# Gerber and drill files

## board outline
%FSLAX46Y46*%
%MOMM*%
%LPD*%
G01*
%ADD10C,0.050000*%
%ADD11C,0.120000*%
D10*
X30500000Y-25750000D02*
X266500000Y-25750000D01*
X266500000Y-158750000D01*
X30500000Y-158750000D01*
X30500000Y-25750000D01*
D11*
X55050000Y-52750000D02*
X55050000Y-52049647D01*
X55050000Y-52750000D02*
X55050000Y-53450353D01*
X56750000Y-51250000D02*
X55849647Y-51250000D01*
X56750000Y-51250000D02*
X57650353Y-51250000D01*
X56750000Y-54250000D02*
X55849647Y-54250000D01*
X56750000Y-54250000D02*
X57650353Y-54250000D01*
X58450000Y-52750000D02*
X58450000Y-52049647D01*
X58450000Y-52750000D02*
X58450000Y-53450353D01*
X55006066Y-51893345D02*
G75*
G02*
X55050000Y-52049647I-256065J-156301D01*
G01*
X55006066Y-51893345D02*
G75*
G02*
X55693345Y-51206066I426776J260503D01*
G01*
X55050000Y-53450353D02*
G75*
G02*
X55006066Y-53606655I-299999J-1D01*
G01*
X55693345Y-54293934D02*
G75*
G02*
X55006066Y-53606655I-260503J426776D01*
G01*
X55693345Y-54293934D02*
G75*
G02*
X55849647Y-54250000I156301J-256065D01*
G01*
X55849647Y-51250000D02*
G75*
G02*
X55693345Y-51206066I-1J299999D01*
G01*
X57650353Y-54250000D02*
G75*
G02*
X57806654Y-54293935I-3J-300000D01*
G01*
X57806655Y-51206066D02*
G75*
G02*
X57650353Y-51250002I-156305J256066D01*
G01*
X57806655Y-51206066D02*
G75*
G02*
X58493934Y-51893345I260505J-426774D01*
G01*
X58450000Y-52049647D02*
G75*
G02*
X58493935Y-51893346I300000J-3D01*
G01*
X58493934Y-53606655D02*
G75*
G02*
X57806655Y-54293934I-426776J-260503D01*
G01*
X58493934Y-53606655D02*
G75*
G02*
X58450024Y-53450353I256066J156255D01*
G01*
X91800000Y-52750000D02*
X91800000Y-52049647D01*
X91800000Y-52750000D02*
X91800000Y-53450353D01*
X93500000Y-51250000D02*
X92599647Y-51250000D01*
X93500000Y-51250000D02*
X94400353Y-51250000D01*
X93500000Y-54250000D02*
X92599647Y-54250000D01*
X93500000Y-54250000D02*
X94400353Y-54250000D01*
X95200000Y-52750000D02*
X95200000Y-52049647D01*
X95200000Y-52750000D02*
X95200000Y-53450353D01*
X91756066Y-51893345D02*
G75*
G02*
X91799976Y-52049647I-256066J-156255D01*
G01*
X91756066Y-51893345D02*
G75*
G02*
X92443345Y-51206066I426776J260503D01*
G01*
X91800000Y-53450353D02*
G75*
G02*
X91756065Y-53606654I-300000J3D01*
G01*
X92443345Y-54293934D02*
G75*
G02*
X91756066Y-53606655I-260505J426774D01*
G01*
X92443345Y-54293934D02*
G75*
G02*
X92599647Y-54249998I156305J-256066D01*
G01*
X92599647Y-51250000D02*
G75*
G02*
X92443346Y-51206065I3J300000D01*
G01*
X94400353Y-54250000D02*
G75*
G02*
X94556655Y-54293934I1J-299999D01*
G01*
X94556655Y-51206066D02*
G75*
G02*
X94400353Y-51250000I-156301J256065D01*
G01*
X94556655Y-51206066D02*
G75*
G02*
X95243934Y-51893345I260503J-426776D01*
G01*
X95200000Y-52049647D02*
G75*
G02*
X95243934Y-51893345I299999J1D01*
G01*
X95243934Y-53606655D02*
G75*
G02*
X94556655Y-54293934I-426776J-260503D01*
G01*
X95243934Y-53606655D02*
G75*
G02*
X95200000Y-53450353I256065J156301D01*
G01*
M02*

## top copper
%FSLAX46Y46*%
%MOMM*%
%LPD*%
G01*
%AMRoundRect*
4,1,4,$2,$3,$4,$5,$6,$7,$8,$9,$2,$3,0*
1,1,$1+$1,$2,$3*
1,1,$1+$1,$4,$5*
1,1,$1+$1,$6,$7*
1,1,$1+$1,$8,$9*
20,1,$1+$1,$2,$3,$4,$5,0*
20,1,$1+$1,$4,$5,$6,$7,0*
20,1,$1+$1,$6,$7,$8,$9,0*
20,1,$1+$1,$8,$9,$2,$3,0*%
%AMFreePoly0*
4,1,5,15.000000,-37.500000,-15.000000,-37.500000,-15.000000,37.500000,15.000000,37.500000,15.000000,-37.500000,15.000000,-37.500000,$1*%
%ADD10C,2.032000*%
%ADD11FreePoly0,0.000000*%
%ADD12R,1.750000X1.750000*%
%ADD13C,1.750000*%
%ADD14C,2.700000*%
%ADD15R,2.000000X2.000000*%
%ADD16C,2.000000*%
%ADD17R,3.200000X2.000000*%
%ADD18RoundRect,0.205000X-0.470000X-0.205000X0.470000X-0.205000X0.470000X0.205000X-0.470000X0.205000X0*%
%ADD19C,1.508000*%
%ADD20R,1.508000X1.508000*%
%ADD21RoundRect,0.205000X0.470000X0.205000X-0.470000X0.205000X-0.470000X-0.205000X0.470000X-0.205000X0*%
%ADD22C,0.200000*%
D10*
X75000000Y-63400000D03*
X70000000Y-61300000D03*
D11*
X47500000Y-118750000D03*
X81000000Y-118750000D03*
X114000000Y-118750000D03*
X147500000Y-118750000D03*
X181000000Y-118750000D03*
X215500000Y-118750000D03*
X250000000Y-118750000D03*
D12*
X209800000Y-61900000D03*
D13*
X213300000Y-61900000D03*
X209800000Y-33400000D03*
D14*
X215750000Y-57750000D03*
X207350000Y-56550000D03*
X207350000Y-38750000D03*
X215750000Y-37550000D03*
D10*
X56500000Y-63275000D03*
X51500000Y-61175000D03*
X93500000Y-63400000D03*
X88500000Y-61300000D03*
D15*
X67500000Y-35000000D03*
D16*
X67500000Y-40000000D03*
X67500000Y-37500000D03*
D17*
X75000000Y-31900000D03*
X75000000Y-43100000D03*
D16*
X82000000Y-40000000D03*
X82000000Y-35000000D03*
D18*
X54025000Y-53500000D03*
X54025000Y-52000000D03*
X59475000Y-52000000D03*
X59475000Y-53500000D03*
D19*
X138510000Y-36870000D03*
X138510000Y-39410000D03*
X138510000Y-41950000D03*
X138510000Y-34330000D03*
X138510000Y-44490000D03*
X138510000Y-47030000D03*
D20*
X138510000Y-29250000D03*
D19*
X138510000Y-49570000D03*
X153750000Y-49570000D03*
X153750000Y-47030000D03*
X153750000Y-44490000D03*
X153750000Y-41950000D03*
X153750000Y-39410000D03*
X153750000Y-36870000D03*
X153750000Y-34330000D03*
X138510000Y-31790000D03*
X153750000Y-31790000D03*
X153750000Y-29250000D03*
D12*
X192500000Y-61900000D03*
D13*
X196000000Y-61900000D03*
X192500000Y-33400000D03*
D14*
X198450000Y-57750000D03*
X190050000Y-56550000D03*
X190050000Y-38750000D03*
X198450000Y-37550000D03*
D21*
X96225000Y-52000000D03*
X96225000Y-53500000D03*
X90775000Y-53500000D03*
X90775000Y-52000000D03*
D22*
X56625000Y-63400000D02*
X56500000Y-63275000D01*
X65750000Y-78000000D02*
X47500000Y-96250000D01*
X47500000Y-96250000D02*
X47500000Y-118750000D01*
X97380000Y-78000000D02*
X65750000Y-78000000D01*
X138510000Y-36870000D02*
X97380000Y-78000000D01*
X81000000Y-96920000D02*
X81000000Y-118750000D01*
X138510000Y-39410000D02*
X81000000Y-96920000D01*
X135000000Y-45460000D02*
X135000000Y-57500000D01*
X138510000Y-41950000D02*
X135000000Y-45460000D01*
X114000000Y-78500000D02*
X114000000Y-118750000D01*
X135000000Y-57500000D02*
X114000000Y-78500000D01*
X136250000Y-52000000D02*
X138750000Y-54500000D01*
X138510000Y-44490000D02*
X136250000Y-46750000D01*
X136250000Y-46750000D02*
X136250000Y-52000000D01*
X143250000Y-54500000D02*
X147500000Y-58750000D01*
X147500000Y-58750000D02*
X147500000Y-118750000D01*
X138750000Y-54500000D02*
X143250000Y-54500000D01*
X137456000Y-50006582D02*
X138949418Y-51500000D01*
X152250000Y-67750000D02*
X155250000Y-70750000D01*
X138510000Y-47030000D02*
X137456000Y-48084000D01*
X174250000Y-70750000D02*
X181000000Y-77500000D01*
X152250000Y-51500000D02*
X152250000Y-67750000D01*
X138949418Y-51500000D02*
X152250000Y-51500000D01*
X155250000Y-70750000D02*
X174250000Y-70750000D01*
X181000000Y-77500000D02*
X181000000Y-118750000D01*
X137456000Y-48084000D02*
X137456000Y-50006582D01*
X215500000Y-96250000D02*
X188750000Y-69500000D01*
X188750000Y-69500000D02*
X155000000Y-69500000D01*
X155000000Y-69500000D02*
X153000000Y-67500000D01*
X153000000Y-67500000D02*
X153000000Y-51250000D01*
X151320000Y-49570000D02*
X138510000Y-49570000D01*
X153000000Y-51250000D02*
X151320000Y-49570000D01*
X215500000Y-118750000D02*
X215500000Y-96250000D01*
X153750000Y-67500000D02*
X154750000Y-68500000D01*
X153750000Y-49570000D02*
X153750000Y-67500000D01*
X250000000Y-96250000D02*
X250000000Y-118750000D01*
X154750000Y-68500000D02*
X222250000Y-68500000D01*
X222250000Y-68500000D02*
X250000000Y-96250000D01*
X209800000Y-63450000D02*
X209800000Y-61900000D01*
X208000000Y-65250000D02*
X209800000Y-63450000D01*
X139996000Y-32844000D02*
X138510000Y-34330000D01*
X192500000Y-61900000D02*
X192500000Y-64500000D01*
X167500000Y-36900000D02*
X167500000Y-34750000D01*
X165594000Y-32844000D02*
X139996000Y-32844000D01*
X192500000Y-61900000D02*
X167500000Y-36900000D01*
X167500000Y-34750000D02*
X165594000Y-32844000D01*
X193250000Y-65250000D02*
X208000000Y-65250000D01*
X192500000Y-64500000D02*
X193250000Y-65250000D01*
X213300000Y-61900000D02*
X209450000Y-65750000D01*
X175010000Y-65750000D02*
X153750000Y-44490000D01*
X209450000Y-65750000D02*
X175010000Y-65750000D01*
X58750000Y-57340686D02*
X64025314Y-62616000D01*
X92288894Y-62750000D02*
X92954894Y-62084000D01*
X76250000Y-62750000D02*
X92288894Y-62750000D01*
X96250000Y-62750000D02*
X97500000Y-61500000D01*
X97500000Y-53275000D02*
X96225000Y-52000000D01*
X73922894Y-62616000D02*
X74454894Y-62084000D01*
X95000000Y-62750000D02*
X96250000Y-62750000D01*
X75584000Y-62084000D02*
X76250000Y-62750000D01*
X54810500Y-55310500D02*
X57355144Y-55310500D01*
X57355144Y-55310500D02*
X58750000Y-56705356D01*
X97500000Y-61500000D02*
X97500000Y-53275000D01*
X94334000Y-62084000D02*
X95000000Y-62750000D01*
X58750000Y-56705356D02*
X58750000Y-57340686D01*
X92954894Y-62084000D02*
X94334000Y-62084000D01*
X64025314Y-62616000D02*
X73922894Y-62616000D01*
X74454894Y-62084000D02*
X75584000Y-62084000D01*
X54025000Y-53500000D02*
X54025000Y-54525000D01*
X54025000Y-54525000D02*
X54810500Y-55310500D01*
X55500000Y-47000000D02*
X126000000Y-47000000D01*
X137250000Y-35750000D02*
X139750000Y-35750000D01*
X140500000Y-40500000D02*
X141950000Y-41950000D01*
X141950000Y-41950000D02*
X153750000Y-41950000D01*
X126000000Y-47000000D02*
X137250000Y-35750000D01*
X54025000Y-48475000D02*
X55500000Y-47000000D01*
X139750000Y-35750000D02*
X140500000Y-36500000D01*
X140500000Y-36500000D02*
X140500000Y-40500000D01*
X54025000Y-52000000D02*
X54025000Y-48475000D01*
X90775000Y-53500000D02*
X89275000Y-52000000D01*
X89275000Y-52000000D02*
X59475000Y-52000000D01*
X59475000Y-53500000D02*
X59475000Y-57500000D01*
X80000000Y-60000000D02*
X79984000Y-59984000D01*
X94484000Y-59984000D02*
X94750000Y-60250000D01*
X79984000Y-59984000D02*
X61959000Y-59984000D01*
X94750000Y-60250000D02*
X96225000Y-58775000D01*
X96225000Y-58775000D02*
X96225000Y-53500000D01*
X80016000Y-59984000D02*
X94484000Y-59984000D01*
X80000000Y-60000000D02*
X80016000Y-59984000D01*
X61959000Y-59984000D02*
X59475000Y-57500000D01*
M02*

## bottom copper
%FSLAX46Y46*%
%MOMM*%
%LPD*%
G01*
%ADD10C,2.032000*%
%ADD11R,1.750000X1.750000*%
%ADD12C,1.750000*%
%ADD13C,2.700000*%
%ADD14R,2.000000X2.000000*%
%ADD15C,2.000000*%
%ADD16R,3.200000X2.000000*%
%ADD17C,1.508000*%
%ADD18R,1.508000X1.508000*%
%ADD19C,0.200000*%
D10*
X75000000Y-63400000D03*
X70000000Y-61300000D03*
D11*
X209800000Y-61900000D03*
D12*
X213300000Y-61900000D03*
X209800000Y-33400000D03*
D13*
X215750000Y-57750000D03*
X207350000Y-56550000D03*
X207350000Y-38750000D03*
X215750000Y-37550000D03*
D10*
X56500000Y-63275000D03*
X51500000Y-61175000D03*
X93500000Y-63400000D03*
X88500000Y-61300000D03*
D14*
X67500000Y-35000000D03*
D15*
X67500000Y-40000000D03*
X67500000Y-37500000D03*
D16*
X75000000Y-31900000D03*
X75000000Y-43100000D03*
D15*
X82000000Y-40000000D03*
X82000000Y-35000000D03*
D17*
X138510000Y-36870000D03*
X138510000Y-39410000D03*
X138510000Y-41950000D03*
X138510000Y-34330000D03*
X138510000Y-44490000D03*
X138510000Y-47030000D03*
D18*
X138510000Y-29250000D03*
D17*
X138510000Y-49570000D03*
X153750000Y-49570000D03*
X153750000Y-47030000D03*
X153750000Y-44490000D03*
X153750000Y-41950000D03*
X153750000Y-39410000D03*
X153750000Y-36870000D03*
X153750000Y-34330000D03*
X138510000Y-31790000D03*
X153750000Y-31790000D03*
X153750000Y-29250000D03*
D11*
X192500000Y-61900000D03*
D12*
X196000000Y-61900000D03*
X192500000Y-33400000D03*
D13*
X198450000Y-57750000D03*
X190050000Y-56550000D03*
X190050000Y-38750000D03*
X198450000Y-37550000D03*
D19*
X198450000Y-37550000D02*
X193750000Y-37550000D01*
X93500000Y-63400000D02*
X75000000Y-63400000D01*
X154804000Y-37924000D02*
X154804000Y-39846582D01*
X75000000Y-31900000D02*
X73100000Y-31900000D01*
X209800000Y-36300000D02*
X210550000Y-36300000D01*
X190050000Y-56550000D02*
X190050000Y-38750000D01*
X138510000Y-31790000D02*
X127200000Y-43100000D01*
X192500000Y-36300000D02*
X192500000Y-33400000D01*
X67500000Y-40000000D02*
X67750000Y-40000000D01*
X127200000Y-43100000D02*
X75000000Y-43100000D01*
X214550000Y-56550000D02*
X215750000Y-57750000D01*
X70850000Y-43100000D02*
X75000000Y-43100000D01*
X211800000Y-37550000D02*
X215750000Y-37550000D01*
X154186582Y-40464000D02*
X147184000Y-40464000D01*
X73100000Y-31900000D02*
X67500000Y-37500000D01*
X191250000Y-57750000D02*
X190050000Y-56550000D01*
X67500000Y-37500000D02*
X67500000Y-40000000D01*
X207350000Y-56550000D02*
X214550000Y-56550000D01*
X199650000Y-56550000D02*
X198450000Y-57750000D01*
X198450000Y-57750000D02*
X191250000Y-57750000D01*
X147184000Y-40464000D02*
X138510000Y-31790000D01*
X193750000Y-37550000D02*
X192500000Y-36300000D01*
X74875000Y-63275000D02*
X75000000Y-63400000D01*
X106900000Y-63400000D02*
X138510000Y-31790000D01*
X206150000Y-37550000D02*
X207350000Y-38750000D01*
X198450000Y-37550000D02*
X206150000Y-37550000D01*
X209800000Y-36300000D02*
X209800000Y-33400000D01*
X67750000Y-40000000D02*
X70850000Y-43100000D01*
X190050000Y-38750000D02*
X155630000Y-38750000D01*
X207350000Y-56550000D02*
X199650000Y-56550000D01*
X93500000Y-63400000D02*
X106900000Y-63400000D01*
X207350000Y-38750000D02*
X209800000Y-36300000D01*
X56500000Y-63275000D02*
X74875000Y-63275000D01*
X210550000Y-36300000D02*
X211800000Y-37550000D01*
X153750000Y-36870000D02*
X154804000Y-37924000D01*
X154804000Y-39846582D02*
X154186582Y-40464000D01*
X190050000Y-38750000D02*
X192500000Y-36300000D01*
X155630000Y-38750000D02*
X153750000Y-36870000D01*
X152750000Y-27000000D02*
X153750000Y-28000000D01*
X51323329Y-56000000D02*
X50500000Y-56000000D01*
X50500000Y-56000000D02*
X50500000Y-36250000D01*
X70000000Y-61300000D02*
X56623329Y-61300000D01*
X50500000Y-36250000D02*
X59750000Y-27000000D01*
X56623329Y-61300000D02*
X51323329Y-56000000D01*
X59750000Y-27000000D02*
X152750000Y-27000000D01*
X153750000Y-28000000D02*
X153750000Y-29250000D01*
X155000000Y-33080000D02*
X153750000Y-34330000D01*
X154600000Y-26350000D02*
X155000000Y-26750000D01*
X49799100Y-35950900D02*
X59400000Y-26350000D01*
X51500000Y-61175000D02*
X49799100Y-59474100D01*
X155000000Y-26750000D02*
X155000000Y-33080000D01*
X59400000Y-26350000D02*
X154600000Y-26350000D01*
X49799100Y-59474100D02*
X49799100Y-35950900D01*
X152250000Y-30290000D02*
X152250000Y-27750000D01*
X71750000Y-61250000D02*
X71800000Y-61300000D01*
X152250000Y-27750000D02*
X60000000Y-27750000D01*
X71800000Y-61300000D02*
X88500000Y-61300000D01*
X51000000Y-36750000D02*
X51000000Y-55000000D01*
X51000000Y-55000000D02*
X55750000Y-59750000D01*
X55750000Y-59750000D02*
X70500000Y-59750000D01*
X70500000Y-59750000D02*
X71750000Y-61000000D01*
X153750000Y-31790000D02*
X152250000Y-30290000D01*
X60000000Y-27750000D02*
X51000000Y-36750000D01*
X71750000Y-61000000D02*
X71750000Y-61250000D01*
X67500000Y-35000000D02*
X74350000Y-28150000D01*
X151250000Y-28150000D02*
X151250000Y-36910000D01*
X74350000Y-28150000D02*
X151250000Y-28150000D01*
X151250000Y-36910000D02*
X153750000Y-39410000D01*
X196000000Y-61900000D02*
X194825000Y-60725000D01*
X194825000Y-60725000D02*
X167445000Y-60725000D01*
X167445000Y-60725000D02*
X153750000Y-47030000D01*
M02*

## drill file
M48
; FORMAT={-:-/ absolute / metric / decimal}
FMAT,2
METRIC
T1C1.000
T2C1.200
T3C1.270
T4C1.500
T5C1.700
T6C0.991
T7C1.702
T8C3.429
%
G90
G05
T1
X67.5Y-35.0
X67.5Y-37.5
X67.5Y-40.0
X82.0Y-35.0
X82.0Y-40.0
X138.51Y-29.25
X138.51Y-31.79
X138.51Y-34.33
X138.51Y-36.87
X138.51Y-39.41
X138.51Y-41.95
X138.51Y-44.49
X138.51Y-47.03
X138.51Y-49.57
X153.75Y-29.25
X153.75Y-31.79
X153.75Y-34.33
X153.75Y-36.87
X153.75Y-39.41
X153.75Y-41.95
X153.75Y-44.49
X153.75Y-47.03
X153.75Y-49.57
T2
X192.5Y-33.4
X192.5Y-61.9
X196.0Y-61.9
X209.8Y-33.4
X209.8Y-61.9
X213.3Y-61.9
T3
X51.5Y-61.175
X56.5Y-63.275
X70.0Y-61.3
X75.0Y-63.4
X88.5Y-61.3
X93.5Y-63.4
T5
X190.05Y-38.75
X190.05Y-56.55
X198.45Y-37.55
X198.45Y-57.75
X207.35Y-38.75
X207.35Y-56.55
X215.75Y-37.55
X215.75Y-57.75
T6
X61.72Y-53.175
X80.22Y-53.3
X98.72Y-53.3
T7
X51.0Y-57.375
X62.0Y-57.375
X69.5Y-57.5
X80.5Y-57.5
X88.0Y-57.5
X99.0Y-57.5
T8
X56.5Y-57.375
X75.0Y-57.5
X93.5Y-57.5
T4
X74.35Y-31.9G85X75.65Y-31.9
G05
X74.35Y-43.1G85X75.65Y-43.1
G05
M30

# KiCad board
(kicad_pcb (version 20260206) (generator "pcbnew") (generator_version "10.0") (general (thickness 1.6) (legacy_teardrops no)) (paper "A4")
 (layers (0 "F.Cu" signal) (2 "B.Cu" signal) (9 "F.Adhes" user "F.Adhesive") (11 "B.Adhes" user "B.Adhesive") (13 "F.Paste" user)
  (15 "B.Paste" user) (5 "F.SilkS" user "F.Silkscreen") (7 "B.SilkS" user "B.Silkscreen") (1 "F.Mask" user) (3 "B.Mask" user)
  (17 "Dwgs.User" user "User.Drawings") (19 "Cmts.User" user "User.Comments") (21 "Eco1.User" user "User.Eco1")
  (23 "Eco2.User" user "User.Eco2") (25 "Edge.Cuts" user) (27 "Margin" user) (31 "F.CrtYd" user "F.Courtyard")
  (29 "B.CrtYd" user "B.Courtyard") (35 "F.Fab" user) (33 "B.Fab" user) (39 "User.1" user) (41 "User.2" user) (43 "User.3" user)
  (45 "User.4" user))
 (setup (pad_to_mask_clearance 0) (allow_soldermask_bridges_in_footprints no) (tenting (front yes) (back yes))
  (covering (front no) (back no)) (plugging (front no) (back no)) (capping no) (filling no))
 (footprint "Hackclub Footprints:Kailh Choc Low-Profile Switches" (layer "F.Cu") (at 75 57.5)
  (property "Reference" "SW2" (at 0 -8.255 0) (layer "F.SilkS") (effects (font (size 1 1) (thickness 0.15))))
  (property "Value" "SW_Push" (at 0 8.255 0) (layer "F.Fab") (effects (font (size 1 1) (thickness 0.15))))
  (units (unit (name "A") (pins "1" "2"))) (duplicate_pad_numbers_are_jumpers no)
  (pad "" np_thru_hole circle (at -5.5 0) (size 1.7018 1.7018) (drill 1.7018) (layers "*.Cu" "*.Mask"))
  (pad "" np_thru_hole circle (at 0 0) (size 3.429 3.429) (drill 3.429) (layers "*.Cu" "*.Mask"))
  (pad "" np_thru_hole circle (at 5.22 -4.2) (size 0.9906 0.9906) (drill 0.9906) (layers "*.Cu" "*.Mask"))
  (pad "" np_thru_hole circle (at 5.5 0) (size 1.7018 1.7018) (drill 1.7018) (layers "*.Cu" "*.Mask"))
  (pad "1" thru_hole circle (at 0 5.9) (size 2.032 2.032) (drill 1.27) (layers "*.Cu" "*.Mask") (remove_unused_layers no) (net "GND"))
  (pad "2" thru_hole circle (at -5 3.8) (size 2.032 2.032) (drill 1.27) (layers "*.Cu" "*.Mask") (remove_unused_layers no) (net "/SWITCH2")))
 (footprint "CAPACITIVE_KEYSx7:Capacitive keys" (layer "F.Cu") (at 147.5 81.25)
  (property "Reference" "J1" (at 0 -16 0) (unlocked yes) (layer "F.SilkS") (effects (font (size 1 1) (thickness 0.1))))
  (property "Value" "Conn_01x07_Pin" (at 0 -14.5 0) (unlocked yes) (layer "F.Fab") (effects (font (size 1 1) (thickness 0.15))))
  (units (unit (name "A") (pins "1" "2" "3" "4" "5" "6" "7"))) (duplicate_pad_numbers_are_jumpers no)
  (pad "1" smd custom (at -100 37.5) (size 30 75) (layers "F.Cu" "F.Mask" "F.Paste") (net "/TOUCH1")
   (options (clearance outline) (anchor rect)) (primitives))
  (pad "2" smd custom (at -66.5 37.5) (size 30 75) (layers "F.Cu" "F.Mask" "F.Paste") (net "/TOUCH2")
   (options (clearance outline) (anchor rect)) (primitives))
  (pad "3" smd custom (at -33.5 37.5) (size 30 75) (layers "F.Cu" "F.Mask" "F.Paste") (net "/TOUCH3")
   (options (clearance outline) (anchor rect)) (primitives))
  (pad "4" smd custom (at 0 37.5) (size 30 75) (layers "F.Cu" "F.Mask" "F.Paste") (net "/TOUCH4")
   (options (clearance outline) (anchor rect)) (primitives))
  (pad "5" smd custom (at 33.5 37.5) (size 30 75) (layers "F.Cu" "F.Mask" "F.Paste") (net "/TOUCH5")
   (options (clearance outline) (anchor rect)) (primitives))
  (pad "6" smd custom (at 68 37.5) (size 30 75) (layers "F.Cu" "F.Mask" "F.Paste") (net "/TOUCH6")
   (options (clearance outline) (anchor rect)) (primitives))
  (pad "7" smd custom (at 102.5 37.5) (size 30 75) (layers "F.Cu" "F.Mask" "F.Paste") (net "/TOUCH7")
   (options (clearance outline) (anchor rect)) (primitives)))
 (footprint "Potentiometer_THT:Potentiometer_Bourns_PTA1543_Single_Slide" (layer "F.Cu") (at 209.8 61.9 90)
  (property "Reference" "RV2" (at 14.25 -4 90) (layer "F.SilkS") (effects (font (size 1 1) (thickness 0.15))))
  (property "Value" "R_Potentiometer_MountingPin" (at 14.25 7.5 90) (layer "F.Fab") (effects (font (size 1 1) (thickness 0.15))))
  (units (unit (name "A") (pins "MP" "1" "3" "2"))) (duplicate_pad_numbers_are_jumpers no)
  (pad "1" thru_hole rect (at 0 0 90) (size 1.75 1.75) (drill 1.2) (layers "*.Cu" "*.Mask") (remove_unused_layers no) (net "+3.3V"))
  (pad "2" thru_hole circle (at 0 3.5 90) (size 1.75 1.75) (drill 1.2) (layers "*.Cu" "*.Mask") (remove_unused_layers no) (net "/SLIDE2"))
  (pad "3" thru_hole circle (at 28.5 0 90) (size 1.75 1.75) (drill 1.2) (layers "*.Cu" "*.Mask") (remove_unused_layers no) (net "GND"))
  (pad "MP" thru_hole circle (at 4.15 5.95 90) (size 2.7 2.7) (drill 1.7) (layers "*.Cu" "*.Mask") (remove_unused_layers no) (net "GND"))
  (pad "MP" thru_hole circle (at 5.35 -2.45 90) (size 2.7 2.7) (drill 1.7) (layers "*.Cu" "*.Mask") (remove_unused_layers no) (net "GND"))
  (pad "MP" thru_hole circle (at 23.15 -2.45 90) (size 2.7 2.7) (drill 1.7) (layers "*.Cu" "*.Mask") (remove_unused_layers no) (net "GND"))
  (pad "MP" thru_hole circle (at 24.35 5.95 90) (size 2.7 2.7) (drill 1.7) (layers "*.Cu" "*.Mask") (remove_unused_layers no) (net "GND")))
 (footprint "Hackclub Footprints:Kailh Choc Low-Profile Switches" (layer "F.Cu") (at 56.5 57.375)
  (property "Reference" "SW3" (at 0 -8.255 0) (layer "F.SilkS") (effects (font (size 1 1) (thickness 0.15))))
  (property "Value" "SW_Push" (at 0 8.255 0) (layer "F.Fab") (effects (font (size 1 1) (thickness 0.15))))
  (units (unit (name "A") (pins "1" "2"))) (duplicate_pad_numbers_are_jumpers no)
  (pad "" np_thru_hole circle (at -5.5 0) (size 1.7018 1.7018) (drill 1.7018) (layers "*.Cu" "*.Mask"))
  (pad "" np_thru_hole circle (at 0 0) (size 3.429 3.429) (drill 3.429) (layers "*.Cu" "*.Mask"))
  (pad "" np_thru_hole circle (at 5.22 -4.2) (size 0.9906 0.9906) (drill 0.9906) (layers "*.Cu" "*.Mask"))
  (pad "" np_thru_hole circle (at 5.5 0) (size 1.7018 1.7018) (drill 1.7018) (layers "*.Cu" "*.Mask"))
  (pad "1" thru_hole circle (at 0 5.9) (size 2.032 2.032) (drill 1.27) (layers "*.Cu" "*.Mask") (remove_unused_layers no) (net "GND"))
  (pad "2" thru_hole circle (at -5 3.8) (size 2.032 2.032) (drill 1.27) (layers "*.Cu" "*.Mask") (remove_unused_layers no) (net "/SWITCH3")))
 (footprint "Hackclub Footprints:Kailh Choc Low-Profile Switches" (layer "F.Cu") (at 93.5 57.5)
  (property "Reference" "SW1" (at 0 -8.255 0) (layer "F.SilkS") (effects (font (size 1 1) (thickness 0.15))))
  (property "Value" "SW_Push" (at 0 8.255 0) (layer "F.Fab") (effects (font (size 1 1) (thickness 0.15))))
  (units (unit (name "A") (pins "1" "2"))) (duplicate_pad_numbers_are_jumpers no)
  (pad "" np_thru_hole circle (at -5.5 0) (size 1.7018 1.7018) (drill 1.7018) (layers "*.Cu" "*.Mask"))
  (pad "" np_thru_hole circle (at 0 0) (size 3.429 3.429) (drill 3.429) (layers "*.Cu" "*.Mask"))
  (pad "" np_thru_hole circle (at 5.22 -4.2) (size 0.9906 0.9906) (drill 0.9906) (layers "*.Cu" "*.Mask"))
  (pad "" np_thru_hole circle (at 5.5 0) (size 1.7018 1.7018) (drill 1.7018) (layers "*.Cu" "*.Mask"))
  (pad "1" thru_hole circle (at 0 5.9) (size 2.032 2.032) (drill 1.27) (layers "*.Cu" "*.Mask") (remove_unused_layers no) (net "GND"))
  (pad "2" thru_hole circle (at -5 3.8) (size 2.032 2.032) (drill 1.27) (layers "*.Cu" "*.Mask") (remove_unused_layers no) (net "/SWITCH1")))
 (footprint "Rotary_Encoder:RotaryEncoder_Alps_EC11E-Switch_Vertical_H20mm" (layer "F.Cu") (at 67.5 35)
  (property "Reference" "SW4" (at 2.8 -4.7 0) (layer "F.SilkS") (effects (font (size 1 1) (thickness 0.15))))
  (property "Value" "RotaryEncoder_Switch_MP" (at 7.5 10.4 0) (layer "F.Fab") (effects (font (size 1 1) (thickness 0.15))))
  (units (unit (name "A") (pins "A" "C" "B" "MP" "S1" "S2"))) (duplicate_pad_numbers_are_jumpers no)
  (pad "A" thru_hole rect (at 0 0) (size 2 2) (drill 1) (layers "*.Cu" "*.Mask") (remove_unused_layers no) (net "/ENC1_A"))
  (pad "B" thru_hole circle (at 0 5) (size 2 2) (drill 1) (layers "*.Cu" "*.Mask") (remove_unused_layers no) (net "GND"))
  (pad "C" thru_hole circle (at 0 2.5) (size 2 2) (drill 1) (layers "*.Cu" "*.Mask") (remove_unused_layers no) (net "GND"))
  (pad "MP" thru_hole rect (at 7.5 -3.1) (size 3.2 2) (drill oval 2.8 1.5) (layers "*.Cu" "*.Mask") (remove_unused_layers no) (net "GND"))
  (pad "MP" thru_hole rect (at 7.5 8.1) (size 3.2 2) (drill oval 2.8 1.5) (layers "*.Cu" "*.Mask") (remove_unused_layers no) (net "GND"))
  (pad "S1" thru_hole circle (at 14.5 5) (size 2 2) (drill 1) (layers "*.Cu" "*.Mask") (remove_unused_layers no)
   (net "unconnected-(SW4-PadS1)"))
  (pad "S2" thru_hole circle (at 14.5 0) (size 2 2) (drill 1) (layers "*.Cu" "*.Mask") (remove_unused_layers no)
   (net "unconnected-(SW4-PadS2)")))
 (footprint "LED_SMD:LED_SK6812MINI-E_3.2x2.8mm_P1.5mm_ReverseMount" (layer "F.Cu") (at 56.75 52.75)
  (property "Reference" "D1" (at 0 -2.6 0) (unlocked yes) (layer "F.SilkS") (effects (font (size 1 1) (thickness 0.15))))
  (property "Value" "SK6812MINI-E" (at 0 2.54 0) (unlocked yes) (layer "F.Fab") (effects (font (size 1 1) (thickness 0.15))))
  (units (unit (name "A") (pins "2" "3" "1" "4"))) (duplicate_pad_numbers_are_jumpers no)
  (fp_line (start -1.7 0) (end -1.7 -0.700353) (stroke (width 0.12) (type solid)) (layer "Edge.Cuts"))
  (fp_line (start -1.7 0) (end -1.7 0.700353) (stroke (width 0.12) (type solid)) (layer "Edge.Cuts"))
  (fp_line (start 0 -1.5) (end -0.900353 -1.5) (stroke (width 0.12) (type solid)) (layer "Edge.Cuts"))
  (fp_line (start 0 -1.5) (end 0.900353 -1.5) (stroke (width 0.12) (type solid)) (layer "Edge.Cuts"))
  (fp_line (start 0 1.5) (end -0.900353 1.5) (stroke (width 0.12) (type solid)) (layer "Edge.Cuts"))
  (fp_line (start 0 1.5) (end 0.900353 1.5) (stroke (width 0.12) (type solid)) (layer "Edge.Cuts"))
  (fp_line (start 1.7 0) (end 1.7 -0.700353) (stroke (width 0.12) (type solid)) (layer "Edge.Cuts"))
  (fp_line (start 1.7 0) (end 1.7 0.700353) (stroke (width 0.12) (type solid)) (layer "Edge.Cuts"))
  (fp_arc (start -1.743934 -0.856655) (mid -1.711192 -0.781532) (end -1.7 -0.700353) (stroke (width 0.12) (type solid)) (layer "Edge.Cuts"))
  (fp_arc (start -1.743934 -0.856655) (mid -1.670711 -1.470711) (end -1.056655 -1.543934) (stroke (width 0.12) (type solid))
   (layer "Edge.Cuts"))
  (fp_arc (start -1.7 0.700353) (mid -1.711192 0.781532) (end -1.743934 0.856655) (stroke (width 0.12) (type solid)) (layer "Edge.Cuts"))
  (fp_arc (start -1.056655 1.543934) (mid -1.670711 1.470711) (end -1.743934 0.856655) (stroke (width 0.12) (type solid))
   (layer "Edge.Cuts"))
  (fp_arc (start -1.056655 1.543934) (mid -0.981532 1.511192) (end -0.900353 1.5) (stroke (width 0.12) (type solid)) (layer "Edge.Cuts"))
  (fp_arc (start -0.900353 -1.5) (mid -0.981532 -1.511192) (end -1.056655 -1.543934) (stroke (width 0.12) (type solid)) (layer "Edge.Cuts"))
  (fp_arc (start 0.900353 1.5) (mid 0.981532 1.511192) (end 1.056655 1.543934) (stroke (width 0.12) (type solid)) (layer "Edge.Cuts"))
  (fp_arc (start 1.056655 -1.543934) (mid 0.981532 -1.511192) (end 0.900353 -1.5) (stroke (width 0.12) (type solid)) (layer "Edge.Cuts"))
  (fp_arc (start 1.056655 -1.543934) (mid 1.670711 -1.470711) (end 1.743934 -0.856655) (stroke (width 0.12) (type solid))
   (layer "Edge.Cuts"))
  (fp_arc (start 1.7 -0.700353) (mid 1.711192 -0.781532) (end 1.743934 -0.856655) (stroke (width 0.12) (type solid)) (layer "Edge.Cuts"))
  (fp_arc (start 1.743934 0.856655) (mid 1.670711 1.470711) (end 1.056655 1.543934) (stroke (width 0.12) (type solid)) (layer "Edge.Cuts"))
  (fp_arc (start 1.743934 0.856655) (mid 1.711192 0.781532) (end 1.7 0.700353) (stroke (width 0.12) (type solid)) (layer "Edge.Cuts"))
  (pad "1" smd roundrect (at -2.725 0.75) (size 1.35 0.82) (layers "F.Cu" "F.Mask" "F.Paste") (roundrect_rratio 0.25) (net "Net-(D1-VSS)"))
  (pad "2" smd roundrect (at -2.725 -0.75) (size 1.35 0.82) (layers "F.Cu" "F.Mask" "F.Paste") (roundrect_rratio 0.25) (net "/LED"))
  (pad "3" smd roundrect (at 2.725 -0.75) (size 1.35 0.82) (layers "F.Cu" "F.Mask" "F.Paste") (roundrect_rratio 0.25) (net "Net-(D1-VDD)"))
  (pad "4" smd roundrect (at 2.725 0.75) (size 1.35 0.82) (layers "F.Cu" "F.Mask" "F.Paste") (roundrect_rratio 0.25) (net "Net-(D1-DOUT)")))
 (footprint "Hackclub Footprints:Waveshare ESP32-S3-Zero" (layer "F.Cu") (at 146.13 39.41)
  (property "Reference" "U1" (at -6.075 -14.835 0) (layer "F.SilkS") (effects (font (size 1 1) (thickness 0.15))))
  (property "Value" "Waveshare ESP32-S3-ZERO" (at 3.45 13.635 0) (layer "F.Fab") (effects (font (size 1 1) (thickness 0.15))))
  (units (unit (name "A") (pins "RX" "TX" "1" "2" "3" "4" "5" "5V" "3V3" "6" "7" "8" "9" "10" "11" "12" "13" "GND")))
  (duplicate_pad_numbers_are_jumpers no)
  (pad "1" thru_hole circle (at -7.62 -2.54) (size 1.508 1.508) (drill 1) (layers "*.Cu" "*.Mask") (remove_unused_layers no) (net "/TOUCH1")
   (solder_mask_margin 0.102))
  (pad "2" thru_hole circle (at -7.62 0) (size 1.508 1.508) (drill 1) (layers "*.Cu" "*.Mask") (remove_unused_layers no) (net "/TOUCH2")
   (solder_mask_margin 0.102))
  (pad "3" thru_hole circle (at -7.62 2.54) (size 1.508 1.508) (drill 1) (layers "*.Cu" "*.Mask") (remove_unused_layers no) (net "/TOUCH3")
   (solder_mask_margin 0.102))
  (pad "3V3" thru_hole circle (at -7.62 -5.08) (size 1.508 1.508) (drill 1) (layers "*.Cu" "*.Mask") (remove_unused_layers no) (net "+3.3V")
   (solder_mask_margin 0.102))
  (pad "4" thru_hole circle (at -7.62 5.08) (size 1.508 1.508) (drill 1) (layers "*.Cu" "*.Mask") (remove_unused_layers no) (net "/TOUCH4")
   (solder_mask_margin 0.102))
  (pad "5" thru_hole circle (at -7.62 7.62) (size 1.508 1.508) (drill 1) (layers "*.Cu" "*.Mask") (remove_unused_layers no) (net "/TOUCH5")
   (solder_mask_margin 0.102))
  (pad "5V" thru_hole rect (at -7.62 -10.16) (size 1.508 1.508) (drill 1) (layers "*.Cu" "*.Mask") (remove_unused_layers no) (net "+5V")
   (solder_mask_margin 0.102))
  (pad "6" thru_hole circle (at -7.62 10.16) (size 1.508 1.508) (drill 1) (layers "*.Cu" "*.Mask") (remove_unused_layers no) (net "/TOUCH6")
   (solder_mask_margin 0.102))
  (pad "7" thru_hole circle (at 7.62 10.16) (size 1.508 1.508) (drill 1) (layers "*.Cu" "*.Mask") (remove_unused_layers no) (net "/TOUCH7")
   (solder_mask_margin 0.102))
  (pad "8" thru_hole circle (at 7.62 7.62) (size 1.508 1.508) (drill 1) (layers "*.Cu" "*.Mask") (remove_unused_layers no) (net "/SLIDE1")
   (solder_mask_margin 0.102))
  (pad "9" thru_hole circle (at 7.62 5.08) (size 1.508 1.508) (drill 1) (layers "*.Cu" "*.Mask") (remove_unused_layers no) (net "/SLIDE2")
   (solder_mask_margin 0.102))
  (pad "10" thru_hole circle (at 7.62 2.54) (size 1.508 1.508) (drill 1) (layers "*.Cu" "*.Mask") (remove_unused_layers no) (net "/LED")
   (solder_mask_margin 0.102))
  (pad "11" thru_hole circle (at 7.62 0) (size 1.508 1.508) (drill 1) (layers "*.Cu" "*.Mask") (remove_unused_layers no) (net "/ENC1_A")
   (solder_mask_margin 0.102))
  (pad "12" thru_hole circle (at 7.62 -2.54) (size 1.508 1.508) (drill 1) (layers "*.Cu" "*.Mask") (remove_unused_layers no) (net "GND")
   (solder_mask_margin 0.102))
  (pad "13" thru_hole circle (at 7.62 -5.08) (size 1.508 1.508) (drill 1) (layers "*.Cu" "*.Mask") (remove_unused_layers no)
   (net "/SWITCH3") (solder_mask_margin 0.102))
  (pad "GND" thru_hole circle (at -7.62 -7.62) (size 1.508 1.508) (drill 1) (layers "*.Cu" "*.Mask") (remove_unused_layers no) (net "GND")
   (solder_mask_margin 0.102))
  (pad "RX" thru_hole circle (at 7.62 -7.62) (size 1.508 1.508) (drill 1) (layers "*.Cu" "*.Mask") (remove_unused_layers no)
   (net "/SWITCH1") (solder_mask_margin 0.102))
  (pad "TX" thru_hole circle (at 7.62 -10.16) (size 1.508 1.508) (drill 1) (layers "*.Cu" "*.Mask") (remove_unused_layers no)
   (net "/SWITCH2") (solder_mask_margin 0.102)))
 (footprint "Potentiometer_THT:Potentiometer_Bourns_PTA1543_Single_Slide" (layer "F.Cu") (at 192.5 61.9 90)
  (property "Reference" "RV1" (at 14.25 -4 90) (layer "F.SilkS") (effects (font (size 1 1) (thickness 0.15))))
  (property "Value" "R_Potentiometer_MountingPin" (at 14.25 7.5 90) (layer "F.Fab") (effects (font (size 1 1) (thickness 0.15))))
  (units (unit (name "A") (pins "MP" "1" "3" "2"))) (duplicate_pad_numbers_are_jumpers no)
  (pad "1" thru_hole rect (at 0 0 90) (size 1.75 1.75) (drill 1.2) (layers "*.Cu" "*.Mask") (remove_unused_layers no) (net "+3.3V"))
  (pad "2" thru_hole circle (at 0 3.5 90) (size 1.75 1.75) (drill 1.2) (layers "*.Cu" "*.Mask") (remove_unused_layers no) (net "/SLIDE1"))
  (pad "3" thru_hole circle (at 28.5 0 90) (size 1.75 1.75) (drill 1.2) (layers "*.Cu" "*.Mask") (remove_unused_layers no) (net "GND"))
  (pad "MP" thru_hole circle (at 4.15 5.95 90) (size 2.7 2.7) (drill 1.7) (layers "*.Cu" "*.Mask") (remove_unused_layers no) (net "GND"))
  (pad "MP" thru_hole circle (at 5.35 -2.45 90) (size 2.7 2.7) (drill 1.7) (layers "*.Cu" "*.Mask") (remove_unused_layers no) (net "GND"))
  (pad "MP" thru_hole circle (at 23.15 -2.45 90) (size 2.7 2.7) (drill 1.7) (layers "*.Cu" "*.Mask") (remove_unused_layers no) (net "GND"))
  (pad "MP" thru_hole circle (at 24.35 5.95 90) (size 2.7 2.7) (drill 1.7) (layers "*.Cu" "*.Mask") (remove_unused_layers no) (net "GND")))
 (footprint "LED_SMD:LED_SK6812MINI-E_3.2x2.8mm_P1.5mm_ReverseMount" (layer "F.Cu") (at 93.5 52.75 180)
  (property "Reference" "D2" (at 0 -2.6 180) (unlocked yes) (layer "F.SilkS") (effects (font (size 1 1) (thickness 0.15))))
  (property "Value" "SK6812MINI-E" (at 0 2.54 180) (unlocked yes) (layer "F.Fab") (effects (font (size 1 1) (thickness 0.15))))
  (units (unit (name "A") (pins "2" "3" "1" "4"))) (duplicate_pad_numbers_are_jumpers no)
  (fp_line (start 1.7 0) (end 1.7 0.700353) (stroke (width 0.12) (type solid)) (layer "Edge.Cuts"))
  (fp_line (start 1.7 0) (end 1.7 -0.700353) (stroke (width 0.12) (type solid)) (layer "Edge.Cuts"))
  (fp_line (start 0 1.5) (end 0.900353 1.5) (stroke (width 0.12) (type solid)) (layer "Edge.Cuts"))
  (fp_line (start 0 1.5) (end -0.900353 1.5) (stroke (width 0.12) (type solid)) (layer "Edge.Cuts"))
  (fp_line (start 0 -1.5) (end 0.900353 -1.5) (stroke (width 0.12) (type solid)) (layer "Edge.Cuts"))
  (fp_line (start 0 -1.5) (end -0.900353 -1.5) (stroke (width 0.12) (type solid)) (layer "Edge.Cuts"))
  (fp_line (start -1.7 0) (end -1.7 0.700353) (stroke (width 0.12) (type solid)) (layer "Edge.Cuts"))
  (fp_line (start -1.7 0) (end -1.7 -0.700353) (stroke (width 0.12) (type solid)) (layer "Edge.Cuts"))
  (fp_arc (start 1.743934 0.856655) (mid 1.711192 0.781532) (end 1.7 0.700353) (stroke (width 0.12) (type solid)) (layer "Edge.Cuts"))
  (fp_arc (start 1.743934 0.856655) (mid 1.670711 1.470711) (end 1.056655 1.543934) (stroke (width 0.12) (type solid)) (layer "Edge.Cuts"))
  (fp_arc (start 1.7 -0.700353) (mid 1.711192 -0.781532) (end 1.743934 -0.856655) (stroke (width 0.12) (type solid)) (layer "Edge.Cuts"))
  (fp_arc (start 1.056655 -1.543934) (mid 1.670711 -1.470711) (end 1.743934 -0.856655) (stroke (width 0.12) (type solid))
   (layer "Edge.Cuts"))
  (fp_arc (start 1.056655 -1.543934) (mid 0.981532 -1.511192) (end 0.900353 -1.5) (stroke (width 0.12) (type solid)) (layer "Edge.Cuts"))
  (fp_arc (start 0.900353 1.5) (mid 0.981532 1.511192) (end 1.056655 1.543934) (stroke (width 0.12) (type solid)) (layer "Edge.Cuts"))
  (fp_arc (start -0.900353 -1.5) (mid -0.981532 -1.511192) (end -1.056655 -1.543934) (stroke (width 0.12) (type solid)) (layer "Edge.Cuts"))
  (fp_arc (start -1.056655 1.543934) (mid -0.981532 1.511192) (end -0.900353 1.5) (stroke (width 0.12) (type solid)) (layer "Edge.Cuts"))
  (fp_arc (start -1.056655 1.543934) (mid -1.670711 1.470711) (end -1.743934 0.856655) (stroke (width 0.12) (type solid))
   (layer "Edge.Cuts"))
  (fp_arc (start -1.7 0.700353) (mid -1.711192 0.781532) (end -1.743934 0.856655) (stroke (width 0.12) (type solid)) (layer "Edge.Cuts"))
  (fp_arc (start -1.743934 -0.856655) (mid -1.670711 -1.470711) (end -1.056655 -1.543934) (stroke (width 0.12) (type solid))
   (layer "Edge.Cuts"))
  (fp_arc (start -1.743934 -0.856655) (mid -1.711192 -0.781532) (end -1.7 -0.700353) (stroke (width 0.12) (type solid)) (layer "Edge.Cuts"))
  (pad "1" smd roundrect (at -2.725 0.75 180) (size 1.35 0.82) (layers "F.Cu" "F.Mask" "F.Paste") (roundrect_rratio 0.25)
   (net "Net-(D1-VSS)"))
  (pad "2" smd roundrect (at -2.725 -0.75 180) (size 1.35 0.82) (layers "F.Cu" "F.Mask" "F.Paste") (roundrect_rratio 0.25)
   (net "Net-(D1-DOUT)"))
  (pad "3" smd roundrect (at 2.725 -0.75 180) (size 1.35 0.82) (layers "F.Cu" "F.Mask" "F.Paste") (roundrect_rratio 0.25)
   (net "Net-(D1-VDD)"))
  (pad "4" smd roundrect (at 2.725 0.75 180) (size 1.35 0.82) (layers "F.Cu" "F.Mask" "F.Paste") (roundrect_rratio 0.25)
   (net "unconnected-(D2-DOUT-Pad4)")))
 (gr_rect (start 30.5 25.75) (end 266.5 158.75) (stroke (width 0.05) (type default)) (fill no) (layer "Edge.Cuts"))
 (segment (start 56.625 63.4) (end 56.5 63.275) (width 0.2) (layer "F.Cu") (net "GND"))
 (segment (start 198.45 37.55) (end 193.75 37.55) (width 0.2) (layer "B.Cu") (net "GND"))
 (segment (start 93.5 63.4) (end 75 63.4) (width 0.2) (layer "B.Cu") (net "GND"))
 (segment (start 154.804 37.924) (end 154.804 39.846582) (width 0.2) (layer "B.Cu") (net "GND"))
 (segment (start 75 31.9) (end 73.1 31.9) (width 0.2) (layer "B.Cu") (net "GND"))
 (segment (start 209.8 36.3) (end 210.55 36.3) (width 0.2) (layer "B.Cu") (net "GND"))
 (segment (start 190.05 56.55) (end 190.05 38.75) (width 0.2) (layer "B.Cu") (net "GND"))
 (segment (start 138.51 31.79) (end 127.2 43.1) (width 0.2) (layer "B.Cu") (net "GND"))
 (segment (start 192.5 36.3) (end 192.5 33.4) (width 0.2) (layer "B.Cu") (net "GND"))
 (segment (start 67.5 40) (end 67.75 40) (width 0.2) (layer "B.Cu") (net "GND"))
 (segment (start 127.2 43.1) (end 75 43.1) (width 0.2) (layer "B.Cu") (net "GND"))
 (segment (start 214.55 56.55) (end 215.75 57.75) (width 0.2) (layer "B.Cu") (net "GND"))
 (segment (start 70.85 43.1) (end 75 43.1) (width 0.2) (layer "B.Cu") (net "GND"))
 (segment (start 211.8 37.55) (end 215.75 37.55) (width 0.2) (layer "B.Cu") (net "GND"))
 (segment (start 154.186582 40.464) (end 147.184 40.464) (width 0.2) (layer "B.Cu") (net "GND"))
 (segment (start 73.1 31.9) (end 67.5 37.5) (width 0.2) (layer "B.Cu") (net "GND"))
 (segment (start 191.25 57.75) (end 190.05 56.55) (width 0.2) (layer "B.Cu") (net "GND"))
 (segment (start 67.5 37.5) (end 67.5 40) (width 0.2) (layer "B.Cu") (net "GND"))
 (segment (start 207.35 56.55) (end 214.55 56.55) (width 0.2) (layer "B.Cu") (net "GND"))
 (segment (start 199.65 56.55) (end 198.45 57.75) (width 0.2) (layer "B.Cu") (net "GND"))
 (segment (start 198.45 57.75) (end 191.25 57.75) (width 0.2) (layer "B.Cu") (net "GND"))
 (segment (start 147.184 40.464) (end 138.51 31.79) (width 0.2) (layer "B.Cu") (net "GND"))
 (segment (start 193.75 37.55) (end 192.5 36.3) (width 0.2) (layer "B.Cu") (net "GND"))
 (segment (start 74.875 63.275) (end 75 63.4) (width 0.2) (layer "B.Cu") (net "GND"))
 (segment (start 106.9 63.4) (end 138.51 31.79) (width 0.2) (layer "B.Cu") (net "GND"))
 (segment (start 206.15 37.55) (end 207.35 38.75) (width 0.2) (layer "B.Cu") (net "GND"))
 (segment (start 198.45 37.55) (end 206.15 37.55) (width 0.2) (layer "B.Cu") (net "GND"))
 (segment (start 209.8 36.3) (end 209.8 33.4) (width 0.2) (layer "B.Cu") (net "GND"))
 (segment (start 67.75 40) (end 70.85 43.1) (width 0.2) (layer "B.Cu") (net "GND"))
 (segment (start 190.05 38.75) (end 155.63 38.75) (width 0.2) (layer "B.Cu") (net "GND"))
 (segment (start 207.35 56.55) (end 199.65 56.55) (width 0.2) (layer "B.Cu") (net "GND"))
 (segment (start 93.5 63.4) (end 106.9 63.4) (width 0.2) (layer "B.Cu") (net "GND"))
 (segment (start 207.35 38.75) (end 209.8 36.3) (width 0.2) (layer "B.Cu") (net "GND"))
 (segment (start 56.5 63.275) (end 74.875 63.275) (width 0.2) (layer "B.Cu") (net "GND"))
 (segment (start 210.55 36.3) (end 211.8 37.55) (width 0.2) (layer "B.Cu") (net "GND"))
 (segment (start 153.75 36.87) (end 154.804 37.924) (width 0.2) (layer "B.Cu") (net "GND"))
 (segment (start 154.804 39.846582) (end 154.186582 40.464) (width 0.2) (layer "B.Cu") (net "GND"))
 (segment (start 190.05 38.75) (end 192.5 36.3) (width 0.2) (layer "B.Cu") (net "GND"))
 (segment (start 155.63 38.75) (end 153.75 36.87) (width 0.2) (layer "B.Cu") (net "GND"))
 (segment (start 152.75 27) (end 153.75 28) (width 0.2) (layer "B.Cu") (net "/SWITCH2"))
 (segment (start 51.323329 56) (end 50.5 56) (width 0.2) (layer "B.Cu") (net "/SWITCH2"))
 (segment (start 50.5 56) (end 50.5 36.25) (width 0.2) (layer "B.Cu") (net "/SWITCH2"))
 (segment (start 70 61.3) (end 56.623329 61.3) (width 0.2) (layer "B.Cu") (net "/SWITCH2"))
 (segment (start 50.5 36.25) (end 59.75 27) (width 0.2) (layer "B.Cu") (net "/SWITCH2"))
 (segment (start 56.623329 61.3) (end 51.323329 56) (width 0.2) (layer "B.Cu") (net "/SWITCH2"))
 (segment (start 59.75 27) (end 152.75 27) (width 0.2) (layer "B.Cu") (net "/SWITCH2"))
 (segment (start 153.75 28) (end 153.75 29.25) (width 0.2) (layer "B.Cu") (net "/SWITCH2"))
 (segment (start 65.75 78) (end 47.5 96.25) (width 0.2) (layer "F.Cu") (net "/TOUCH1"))
 (segment (start 47.5 96.25) (end 47.5 118.75) (width 0.2) (layer "F.Cu") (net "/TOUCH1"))
 (segment (start 97.38 78) (end 65.75 78) (width 0.2) (layer "F.Cu") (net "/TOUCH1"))
 (segment (start 138.51 36.87) (end 97.38 78) (width 0.2) (layer "F.Cu") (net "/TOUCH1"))
 (segment (start 81 96.92) (end 81 118.75) (width 0.2) (layer "F.Cu") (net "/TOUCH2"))
 (segment (start 138.51 39.41) (end 81 96.92) (width 0.2) (layer "F.Cu") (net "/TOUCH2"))
 (segment (start 135 45.46) (end 135 57.5) (width 0.2) (layer "F.Cu") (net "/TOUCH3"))
 (segment (start 138.51 41.95) (end 135 45.46) (width 0.2) (layer "F.Cu") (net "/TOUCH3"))
 (segment (start 114 78.5) (end 114 118.75) (width 0.2) (layer "F.Cu") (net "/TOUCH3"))
 (segment (start 135 57.5) (end 114 78.5) (width 0.2) (layer "F.Cu") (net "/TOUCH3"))
 (segment (start 136.25 52) (end 138.75 54.5) (width 0.2) (layer "F.Cu") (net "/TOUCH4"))
 (segment (start 138.51 44.49) (end 136.25 46.75) (width 0.2) (layer "F.Cu") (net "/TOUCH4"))
 (segment (start 136.25 46.75) (end 136.25 52) (width 0.2) (layer "F.Cu") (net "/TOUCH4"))
 (segment (start 143.25 54.5) (end 147.5 58.75) (width 0.2) (layer "F.Cu") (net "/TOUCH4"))
 (segment (start 147.5 58.75) (end 147.5 118.75) (width 0.2) (layer "F.Cu") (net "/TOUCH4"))
 (segment (start 138.75 54.5) (end 143.25 54.5) (width 0.2) (layer "F.Cu") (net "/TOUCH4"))
 (segment (start 137.456 50.006582) (end 138.949418 51.5) (width 0.2) (layer "F.Cu") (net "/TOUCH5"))
 (segment (start 152.25 67.75) (end 155.25 70.75) (width 0.2) (layer "F.Cu") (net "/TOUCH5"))
 (segment (start 138.51 47.03) (end 137.456 48.084) (width 0.2) (layer "F.Cu") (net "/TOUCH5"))
 (segment (start 174.25 70.75) (end 181 77.5) (width 0.2) (layer "F.Cu") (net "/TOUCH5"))
 (segment (start 152.25 51.5) (end 152.25 67.75) (width 0.2) (layer "F.Cu") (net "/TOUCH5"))
 (segment (start 138.949418 51.5) (end 152.25 51.5) (width 0.2) (layer "F.Cu") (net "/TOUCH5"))
 (segment (start 155.25 70.75) (end 174.25 70.75) (width 0.2) (layer "F.Cu") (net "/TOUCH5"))
 (segment (start 181 77.5) (end 181 118.75) (width 0.2) (layer "F.Cu") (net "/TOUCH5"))
 (segment (start 137.456 48.084) (end 137.456 50.006582) (width 0.2) (layer "F.Cu") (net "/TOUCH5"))
 (segment (start 215.5 96.25) (end 188.75 69.5) (width 0.2) (layer "F.Cu") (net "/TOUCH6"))
 (segment (start 188.75 69.5) (end 155 69.5) (width 0.2) (layer "F.Cu") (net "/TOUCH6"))
 (segment (start 155 69.5) (end 153 67.5) (width 0.2) (layer "F.Cu") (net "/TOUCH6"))
 (segment (start 153 67.5) (end 153 51.25) (width 0.2) (layer "F.Cu") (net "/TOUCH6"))
 (segment (start 151.32 49.57) (end 138.51 49.57) (width 0.2) (layer "F.Cu") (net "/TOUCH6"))
 (segment (start 153 51.25) (end 151.32 49.57) (width 0.2) (layer "F.Cu") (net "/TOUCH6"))
 (segment (start 215.5 118.75) (end 215.5 96.25) (width 0.2) (layer "F.Cu") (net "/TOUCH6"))
 (segment (start 153.75 67.5) (end 154.75 68.5) (width 0.2) (layer "F.Cu") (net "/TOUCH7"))
 (segment (start 153.75 49.57) (end 153.75 67.5) (width 0.2) (layer "F.Cu") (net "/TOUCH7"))
 (segment (start 250 96.25) (end 250 118.75) (width 0.2) (layer "F.Cu") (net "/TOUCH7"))
 (segment (start 154.75 68.5) (end 222.25 68.5) (width 0.2) (layer "F.Cu") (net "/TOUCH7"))
 (segment (start 222.25 68.5) (end 250 96.25) (width 0.2) (layer "F.Cu") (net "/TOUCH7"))
 (segment (start 209.8 63.45) (end 209.8 61.9) (width 0.2) (layer "F.Cu") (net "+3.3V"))
 (segment (start 208 65.25) (end 209.8 63.45) (width 0.2) (layer "F.Cu") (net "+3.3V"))
 (segment (start 139.996 32.844) (end 138.51 34.33) (width 0.2) (layer "F.Cu") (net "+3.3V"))
 (segment (start 192.5 61.9) (end 192.5 64.5) (width 0.2) (layer "F.Cu") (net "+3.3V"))
 (segment (start 167.5 36.9) (end 167.5 34.75) (width 0.2) (layer "F.Cu") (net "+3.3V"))
 (segment (start 165.594 32.844) (end 139.996 32.844) (width 0.2) (layer "F.Cu") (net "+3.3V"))
 (segment (start 192.5 61.9) (end 167.5 36.9) (width 0.2) (layer "F.Cu") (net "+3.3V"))
 (segment (start 167.5 34.75) (end 165.594 32.844) (width 0.2) (layer "F.Cu") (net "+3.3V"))
 (segment (start 193.25 65.25) (end 208 65.25) (width 0.2) (layer "F.Cu") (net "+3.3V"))
 (segment (start 192.5 64.5) (end 193.25 65.25) (width 0.2) (layer "F.Cu") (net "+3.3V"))
 (segment (start 213.3 61.9) (end 209.45 65.75) (width 0.2) (layer "F.Cu") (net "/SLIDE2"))
 (segment (start 175.01 65.75) (end 153.75 44.49) (width 0.2) (layer "F.Cu") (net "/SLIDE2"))
 (segment (start 209.45 65.75) (end 175.01 65.75) (width 0.2) (layer "F.Cu") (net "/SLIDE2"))
 (segment (start 155 33.08) (end 153.75 34.33) (width 0.2) (layer "B.Cu") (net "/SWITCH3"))
 (segment (start 154.6 26.35) (end 155 26.75) (width 0.2) (layer "B.Cu") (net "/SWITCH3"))
 (segment (start 49.7991 35.9509) (end 59.4 26.35) (width 0.2) (layer "B.Cu") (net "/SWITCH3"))
 (segment (start 51.5 61.175) (end 49.7991 59.4741) (width 0.2) (layer "B.Cu") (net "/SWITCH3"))
 (segment (start 155 26.75) (end 155 33.08) (width 0.2) (layer "B.Cu") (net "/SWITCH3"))
 (segment (start 59.4 26.35) (end 154.6 26.35) (width 0.2) (layer "B.Cu") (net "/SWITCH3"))
 (segment (start 49.7991 59.4741) (end 49.7991 35.9509) (width 0.2) (layer "B.Cu") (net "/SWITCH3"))
 (segment (start 152.25 30.29) (end 152.25 27.75) (width 0.2) (layer "B.Cu") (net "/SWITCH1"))
 (segment (start 71.75 61.25) (end 71.8 61.3) (width 0.2) (layer "B.Cu") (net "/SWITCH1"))
 (segment (start 152.25 27.75) (end 60 27.75) (width 0.2) (layer "B.Cu") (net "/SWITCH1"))
 (segment (start 71.8 61.3) (end 88.5 61.3) (width 0.2) (layer "B.Cu") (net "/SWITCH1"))
 (segment (start 51 36.75) (end 51 55) (width 0.2) (layer "B.Cu") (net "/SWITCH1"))
 (segment (start 51 55) (end 55.75 59.75) (width 0.2) (layer "B.Cu") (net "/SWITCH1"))
 (segment (start 55.75 59.75) (end 70.5 59.75) (width 0.2) (layer "B.Cu") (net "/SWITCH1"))
 (segment (start 70.5 59.75) (end 71.75 61) (width 0.2) (layer "B.Cu") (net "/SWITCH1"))
 (segment (start 153.75 31.79) (end 152.25 30.29) (width 0.2) (layer "B.Cu") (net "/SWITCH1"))
 (segment (start 60 27.75) (end 51 36.75) (width 0.2) (layer "B.Cu") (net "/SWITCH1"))
 (segment (start 71.75 61) (end 71.75 61.25) (width 0.2) (layer "B.Cu") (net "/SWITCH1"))
 (segment (start 67.5 35) (end 74.35 28.15) (width 0.2) (layer "B.Cu") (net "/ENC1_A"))
 (segment (start 151.25 28.15) (end 151.25 36.91) (width 0.2) (layer "B.Cu") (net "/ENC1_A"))
 (segment (start 74.35 28.15) (end 151.25 28.15) (width 0.2) (layer "B.Cu") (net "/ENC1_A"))
 (segment (start 151.25 36.91) (end 153.75 39.41) (width 0.2) (layer "B.Cu") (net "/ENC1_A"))
 (segment (start 58.75 57.340686) (end 64.025314 62.616) (width 0.2) (layer "F.Cu") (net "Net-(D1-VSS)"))
 (segment (start 92.288894 62.75) (end 92.954894 62.084) (width 0.2) (layer "F.Cu") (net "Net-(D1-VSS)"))
 (segment (start 76.25 62.75) (end 92.288894 62.75) (width 0.2) (layer "F.Cu") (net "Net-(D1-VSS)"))
 (segment (start 96.25 62.75) (end 97.5 61.5) (width 0.2) (layer "F.Cu") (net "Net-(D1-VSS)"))
 (segment (start 97.5 53.275) (end 96.225 52) (width 0.2) (layer "F.Cu") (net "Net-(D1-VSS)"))
 (segment (start 73.922894 62.616) (end 74.454894 62.084) (width 0.2) (layer "F.Cu") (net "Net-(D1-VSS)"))
 (segment (start 95 62.75) (end 96.25 62.75) (width 0.2) (layer "F.Cu") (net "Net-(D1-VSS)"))
 (segment (start 75.584 62.084) (end 76.25 62.75) (width 0.2) (layer "F.Cu") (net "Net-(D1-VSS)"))
 (segment (start 54.8105 55.3105) (end 57.355144 55.3105) (width 0.2) (layer "F.Cu") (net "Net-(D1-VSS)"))
 (segment (start 57.355144 55.3105) (end 58.75 56.705356) (width 0.2) (layer "F.Cu") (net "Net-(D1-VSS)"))
 (segment (start 97.5 61.5) (end 97.5 53.275) (width 0.2) (layer "F.Cu") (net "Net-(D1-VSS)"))
 (segment (start 94.334 62.084) (end 95 62.75) (width 0.2) (layer "F.Cu") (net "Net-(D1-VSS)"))
 (segment (start 58.75 56.705356) (end 58.75 57.340686) (width 0.2) (layer "F.Cu") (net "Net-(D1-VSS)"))
 (segment (start 92.954894 62.084) (end 94.334 62.084) (width 0.2) (layer "F.Cu") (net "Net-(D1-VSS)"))
 (segment (start 64.025314 62.616) (end 73.922894 62.616) (width 0.2) (layer "F.Cu") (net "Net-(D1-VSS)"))
 (segment (start 74.454894 62.084) (end 75.584 62.084) (width 0.2) (layer "F.Cu") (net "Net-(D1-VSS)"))
 (segment (start 54.025 53.5) (end 54.025 54.525) (width 0.2) (layer "F.Cu") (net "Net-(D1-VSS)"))
 (segment (start 54.025 54.525) (end 54.8105 55.3105) (width 0.2) (layer "F.Cu") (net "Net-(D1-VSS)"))
 (segment (start 55.5 47) (end 126 47) (width 0.2) (layer "F.Cu") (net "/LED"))
 (segment (start 137.25 35.75) (end 139.75 35.75) (width 0.2) (layer "F.Cu") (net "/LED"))
 (segment (start 140.5 40.5) (end 141.95 41.95) (width 0.2) (layer "F.Cu") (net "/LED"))
 (segment (start 141.95 41.95) (end 153.75 41.95) (width 0.2) (layer "F.Cu") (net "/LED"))
 (segment (start 126 47) (end 137.25 35.75) (width 0.2) (layer "F.Cu") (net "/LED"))
 (segment (start 54.025 48.475) (end 55.5 47) (width 0.2) (layer "F.Cu") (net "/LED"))
 (segment (start 139.75 35.75) (end 140.5 36.5) (width 0.2) (layer "F.Cu") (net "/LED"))
 (segment (start 140.5 36.5) (end 140.5 40.5) (width 0.2) (layer "F.Cu") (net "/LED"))
 (segment (start 54.025 52) (end 54.025 48.475) (width 0.2) (layer "F.Cu") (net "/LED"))
 (segment (start 90.775 53.5) (end 89.275 52) (width 0.2) (layer "F.Cu") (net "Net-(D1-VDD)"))
 (segment (start 89.275 52) (end 59.475 52) (width 0.2) (layer "F.Cu") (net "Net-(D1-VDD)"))
 (segment (start 59.475 53.5) (end 59.475 57.5) (width 0.2) (layer "F.Cu") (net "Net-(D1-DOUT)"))
 (segment (start 80 60) (end 79.984 59.984) (width 0.2) (layer "F.Cu") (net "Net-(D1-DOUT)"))
 (segment (start 94.484 59.984) (end 94.75 60.25) (width 0.2) (layer "F.Cu") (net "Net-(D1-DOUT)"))
 (segment (start 79.984 59.984) (end 61.959 59.984) (width 0.2) (layer "F.Cu") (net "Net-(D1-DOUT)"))
 (segment (start 94.75 60.25) (end 96.225 58.775) (width 0.2) (layer "F.Cu") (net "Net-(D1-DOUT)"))
 (segment (start 96.225 58.775) (end 96.225 53.5) (width 0.2) (layer "F.Cu") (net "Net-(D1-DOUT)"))
 (segment (start 80.016 59.984) (end 94.484 59.984) (width 0.2) (layer "F.Cu") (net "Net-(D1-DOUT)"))
 (segment (start 80 60) (end 80.016 59.984) (width 0.2) (layer "F.Cu") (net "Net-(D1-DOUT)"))
 (segment (start 61.959 59.984) (end 59.475 57.5) (width 0.2) (layer "F.Cu") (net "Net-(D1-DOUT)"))
 (segment (start 196 61.9) (end 194.825 60.725) (width 0.2) (layer "B.Cu") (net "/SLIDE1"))
 (segment (start 194.825 60.725) (end 167.445 60.725) (width 0.2) (layer "B.Cu") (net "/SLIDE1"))
 (segment (start 167.445 60.725) (end 153.75 47.03) (width 0.2) (layer "B.Cu") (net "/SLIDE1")))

